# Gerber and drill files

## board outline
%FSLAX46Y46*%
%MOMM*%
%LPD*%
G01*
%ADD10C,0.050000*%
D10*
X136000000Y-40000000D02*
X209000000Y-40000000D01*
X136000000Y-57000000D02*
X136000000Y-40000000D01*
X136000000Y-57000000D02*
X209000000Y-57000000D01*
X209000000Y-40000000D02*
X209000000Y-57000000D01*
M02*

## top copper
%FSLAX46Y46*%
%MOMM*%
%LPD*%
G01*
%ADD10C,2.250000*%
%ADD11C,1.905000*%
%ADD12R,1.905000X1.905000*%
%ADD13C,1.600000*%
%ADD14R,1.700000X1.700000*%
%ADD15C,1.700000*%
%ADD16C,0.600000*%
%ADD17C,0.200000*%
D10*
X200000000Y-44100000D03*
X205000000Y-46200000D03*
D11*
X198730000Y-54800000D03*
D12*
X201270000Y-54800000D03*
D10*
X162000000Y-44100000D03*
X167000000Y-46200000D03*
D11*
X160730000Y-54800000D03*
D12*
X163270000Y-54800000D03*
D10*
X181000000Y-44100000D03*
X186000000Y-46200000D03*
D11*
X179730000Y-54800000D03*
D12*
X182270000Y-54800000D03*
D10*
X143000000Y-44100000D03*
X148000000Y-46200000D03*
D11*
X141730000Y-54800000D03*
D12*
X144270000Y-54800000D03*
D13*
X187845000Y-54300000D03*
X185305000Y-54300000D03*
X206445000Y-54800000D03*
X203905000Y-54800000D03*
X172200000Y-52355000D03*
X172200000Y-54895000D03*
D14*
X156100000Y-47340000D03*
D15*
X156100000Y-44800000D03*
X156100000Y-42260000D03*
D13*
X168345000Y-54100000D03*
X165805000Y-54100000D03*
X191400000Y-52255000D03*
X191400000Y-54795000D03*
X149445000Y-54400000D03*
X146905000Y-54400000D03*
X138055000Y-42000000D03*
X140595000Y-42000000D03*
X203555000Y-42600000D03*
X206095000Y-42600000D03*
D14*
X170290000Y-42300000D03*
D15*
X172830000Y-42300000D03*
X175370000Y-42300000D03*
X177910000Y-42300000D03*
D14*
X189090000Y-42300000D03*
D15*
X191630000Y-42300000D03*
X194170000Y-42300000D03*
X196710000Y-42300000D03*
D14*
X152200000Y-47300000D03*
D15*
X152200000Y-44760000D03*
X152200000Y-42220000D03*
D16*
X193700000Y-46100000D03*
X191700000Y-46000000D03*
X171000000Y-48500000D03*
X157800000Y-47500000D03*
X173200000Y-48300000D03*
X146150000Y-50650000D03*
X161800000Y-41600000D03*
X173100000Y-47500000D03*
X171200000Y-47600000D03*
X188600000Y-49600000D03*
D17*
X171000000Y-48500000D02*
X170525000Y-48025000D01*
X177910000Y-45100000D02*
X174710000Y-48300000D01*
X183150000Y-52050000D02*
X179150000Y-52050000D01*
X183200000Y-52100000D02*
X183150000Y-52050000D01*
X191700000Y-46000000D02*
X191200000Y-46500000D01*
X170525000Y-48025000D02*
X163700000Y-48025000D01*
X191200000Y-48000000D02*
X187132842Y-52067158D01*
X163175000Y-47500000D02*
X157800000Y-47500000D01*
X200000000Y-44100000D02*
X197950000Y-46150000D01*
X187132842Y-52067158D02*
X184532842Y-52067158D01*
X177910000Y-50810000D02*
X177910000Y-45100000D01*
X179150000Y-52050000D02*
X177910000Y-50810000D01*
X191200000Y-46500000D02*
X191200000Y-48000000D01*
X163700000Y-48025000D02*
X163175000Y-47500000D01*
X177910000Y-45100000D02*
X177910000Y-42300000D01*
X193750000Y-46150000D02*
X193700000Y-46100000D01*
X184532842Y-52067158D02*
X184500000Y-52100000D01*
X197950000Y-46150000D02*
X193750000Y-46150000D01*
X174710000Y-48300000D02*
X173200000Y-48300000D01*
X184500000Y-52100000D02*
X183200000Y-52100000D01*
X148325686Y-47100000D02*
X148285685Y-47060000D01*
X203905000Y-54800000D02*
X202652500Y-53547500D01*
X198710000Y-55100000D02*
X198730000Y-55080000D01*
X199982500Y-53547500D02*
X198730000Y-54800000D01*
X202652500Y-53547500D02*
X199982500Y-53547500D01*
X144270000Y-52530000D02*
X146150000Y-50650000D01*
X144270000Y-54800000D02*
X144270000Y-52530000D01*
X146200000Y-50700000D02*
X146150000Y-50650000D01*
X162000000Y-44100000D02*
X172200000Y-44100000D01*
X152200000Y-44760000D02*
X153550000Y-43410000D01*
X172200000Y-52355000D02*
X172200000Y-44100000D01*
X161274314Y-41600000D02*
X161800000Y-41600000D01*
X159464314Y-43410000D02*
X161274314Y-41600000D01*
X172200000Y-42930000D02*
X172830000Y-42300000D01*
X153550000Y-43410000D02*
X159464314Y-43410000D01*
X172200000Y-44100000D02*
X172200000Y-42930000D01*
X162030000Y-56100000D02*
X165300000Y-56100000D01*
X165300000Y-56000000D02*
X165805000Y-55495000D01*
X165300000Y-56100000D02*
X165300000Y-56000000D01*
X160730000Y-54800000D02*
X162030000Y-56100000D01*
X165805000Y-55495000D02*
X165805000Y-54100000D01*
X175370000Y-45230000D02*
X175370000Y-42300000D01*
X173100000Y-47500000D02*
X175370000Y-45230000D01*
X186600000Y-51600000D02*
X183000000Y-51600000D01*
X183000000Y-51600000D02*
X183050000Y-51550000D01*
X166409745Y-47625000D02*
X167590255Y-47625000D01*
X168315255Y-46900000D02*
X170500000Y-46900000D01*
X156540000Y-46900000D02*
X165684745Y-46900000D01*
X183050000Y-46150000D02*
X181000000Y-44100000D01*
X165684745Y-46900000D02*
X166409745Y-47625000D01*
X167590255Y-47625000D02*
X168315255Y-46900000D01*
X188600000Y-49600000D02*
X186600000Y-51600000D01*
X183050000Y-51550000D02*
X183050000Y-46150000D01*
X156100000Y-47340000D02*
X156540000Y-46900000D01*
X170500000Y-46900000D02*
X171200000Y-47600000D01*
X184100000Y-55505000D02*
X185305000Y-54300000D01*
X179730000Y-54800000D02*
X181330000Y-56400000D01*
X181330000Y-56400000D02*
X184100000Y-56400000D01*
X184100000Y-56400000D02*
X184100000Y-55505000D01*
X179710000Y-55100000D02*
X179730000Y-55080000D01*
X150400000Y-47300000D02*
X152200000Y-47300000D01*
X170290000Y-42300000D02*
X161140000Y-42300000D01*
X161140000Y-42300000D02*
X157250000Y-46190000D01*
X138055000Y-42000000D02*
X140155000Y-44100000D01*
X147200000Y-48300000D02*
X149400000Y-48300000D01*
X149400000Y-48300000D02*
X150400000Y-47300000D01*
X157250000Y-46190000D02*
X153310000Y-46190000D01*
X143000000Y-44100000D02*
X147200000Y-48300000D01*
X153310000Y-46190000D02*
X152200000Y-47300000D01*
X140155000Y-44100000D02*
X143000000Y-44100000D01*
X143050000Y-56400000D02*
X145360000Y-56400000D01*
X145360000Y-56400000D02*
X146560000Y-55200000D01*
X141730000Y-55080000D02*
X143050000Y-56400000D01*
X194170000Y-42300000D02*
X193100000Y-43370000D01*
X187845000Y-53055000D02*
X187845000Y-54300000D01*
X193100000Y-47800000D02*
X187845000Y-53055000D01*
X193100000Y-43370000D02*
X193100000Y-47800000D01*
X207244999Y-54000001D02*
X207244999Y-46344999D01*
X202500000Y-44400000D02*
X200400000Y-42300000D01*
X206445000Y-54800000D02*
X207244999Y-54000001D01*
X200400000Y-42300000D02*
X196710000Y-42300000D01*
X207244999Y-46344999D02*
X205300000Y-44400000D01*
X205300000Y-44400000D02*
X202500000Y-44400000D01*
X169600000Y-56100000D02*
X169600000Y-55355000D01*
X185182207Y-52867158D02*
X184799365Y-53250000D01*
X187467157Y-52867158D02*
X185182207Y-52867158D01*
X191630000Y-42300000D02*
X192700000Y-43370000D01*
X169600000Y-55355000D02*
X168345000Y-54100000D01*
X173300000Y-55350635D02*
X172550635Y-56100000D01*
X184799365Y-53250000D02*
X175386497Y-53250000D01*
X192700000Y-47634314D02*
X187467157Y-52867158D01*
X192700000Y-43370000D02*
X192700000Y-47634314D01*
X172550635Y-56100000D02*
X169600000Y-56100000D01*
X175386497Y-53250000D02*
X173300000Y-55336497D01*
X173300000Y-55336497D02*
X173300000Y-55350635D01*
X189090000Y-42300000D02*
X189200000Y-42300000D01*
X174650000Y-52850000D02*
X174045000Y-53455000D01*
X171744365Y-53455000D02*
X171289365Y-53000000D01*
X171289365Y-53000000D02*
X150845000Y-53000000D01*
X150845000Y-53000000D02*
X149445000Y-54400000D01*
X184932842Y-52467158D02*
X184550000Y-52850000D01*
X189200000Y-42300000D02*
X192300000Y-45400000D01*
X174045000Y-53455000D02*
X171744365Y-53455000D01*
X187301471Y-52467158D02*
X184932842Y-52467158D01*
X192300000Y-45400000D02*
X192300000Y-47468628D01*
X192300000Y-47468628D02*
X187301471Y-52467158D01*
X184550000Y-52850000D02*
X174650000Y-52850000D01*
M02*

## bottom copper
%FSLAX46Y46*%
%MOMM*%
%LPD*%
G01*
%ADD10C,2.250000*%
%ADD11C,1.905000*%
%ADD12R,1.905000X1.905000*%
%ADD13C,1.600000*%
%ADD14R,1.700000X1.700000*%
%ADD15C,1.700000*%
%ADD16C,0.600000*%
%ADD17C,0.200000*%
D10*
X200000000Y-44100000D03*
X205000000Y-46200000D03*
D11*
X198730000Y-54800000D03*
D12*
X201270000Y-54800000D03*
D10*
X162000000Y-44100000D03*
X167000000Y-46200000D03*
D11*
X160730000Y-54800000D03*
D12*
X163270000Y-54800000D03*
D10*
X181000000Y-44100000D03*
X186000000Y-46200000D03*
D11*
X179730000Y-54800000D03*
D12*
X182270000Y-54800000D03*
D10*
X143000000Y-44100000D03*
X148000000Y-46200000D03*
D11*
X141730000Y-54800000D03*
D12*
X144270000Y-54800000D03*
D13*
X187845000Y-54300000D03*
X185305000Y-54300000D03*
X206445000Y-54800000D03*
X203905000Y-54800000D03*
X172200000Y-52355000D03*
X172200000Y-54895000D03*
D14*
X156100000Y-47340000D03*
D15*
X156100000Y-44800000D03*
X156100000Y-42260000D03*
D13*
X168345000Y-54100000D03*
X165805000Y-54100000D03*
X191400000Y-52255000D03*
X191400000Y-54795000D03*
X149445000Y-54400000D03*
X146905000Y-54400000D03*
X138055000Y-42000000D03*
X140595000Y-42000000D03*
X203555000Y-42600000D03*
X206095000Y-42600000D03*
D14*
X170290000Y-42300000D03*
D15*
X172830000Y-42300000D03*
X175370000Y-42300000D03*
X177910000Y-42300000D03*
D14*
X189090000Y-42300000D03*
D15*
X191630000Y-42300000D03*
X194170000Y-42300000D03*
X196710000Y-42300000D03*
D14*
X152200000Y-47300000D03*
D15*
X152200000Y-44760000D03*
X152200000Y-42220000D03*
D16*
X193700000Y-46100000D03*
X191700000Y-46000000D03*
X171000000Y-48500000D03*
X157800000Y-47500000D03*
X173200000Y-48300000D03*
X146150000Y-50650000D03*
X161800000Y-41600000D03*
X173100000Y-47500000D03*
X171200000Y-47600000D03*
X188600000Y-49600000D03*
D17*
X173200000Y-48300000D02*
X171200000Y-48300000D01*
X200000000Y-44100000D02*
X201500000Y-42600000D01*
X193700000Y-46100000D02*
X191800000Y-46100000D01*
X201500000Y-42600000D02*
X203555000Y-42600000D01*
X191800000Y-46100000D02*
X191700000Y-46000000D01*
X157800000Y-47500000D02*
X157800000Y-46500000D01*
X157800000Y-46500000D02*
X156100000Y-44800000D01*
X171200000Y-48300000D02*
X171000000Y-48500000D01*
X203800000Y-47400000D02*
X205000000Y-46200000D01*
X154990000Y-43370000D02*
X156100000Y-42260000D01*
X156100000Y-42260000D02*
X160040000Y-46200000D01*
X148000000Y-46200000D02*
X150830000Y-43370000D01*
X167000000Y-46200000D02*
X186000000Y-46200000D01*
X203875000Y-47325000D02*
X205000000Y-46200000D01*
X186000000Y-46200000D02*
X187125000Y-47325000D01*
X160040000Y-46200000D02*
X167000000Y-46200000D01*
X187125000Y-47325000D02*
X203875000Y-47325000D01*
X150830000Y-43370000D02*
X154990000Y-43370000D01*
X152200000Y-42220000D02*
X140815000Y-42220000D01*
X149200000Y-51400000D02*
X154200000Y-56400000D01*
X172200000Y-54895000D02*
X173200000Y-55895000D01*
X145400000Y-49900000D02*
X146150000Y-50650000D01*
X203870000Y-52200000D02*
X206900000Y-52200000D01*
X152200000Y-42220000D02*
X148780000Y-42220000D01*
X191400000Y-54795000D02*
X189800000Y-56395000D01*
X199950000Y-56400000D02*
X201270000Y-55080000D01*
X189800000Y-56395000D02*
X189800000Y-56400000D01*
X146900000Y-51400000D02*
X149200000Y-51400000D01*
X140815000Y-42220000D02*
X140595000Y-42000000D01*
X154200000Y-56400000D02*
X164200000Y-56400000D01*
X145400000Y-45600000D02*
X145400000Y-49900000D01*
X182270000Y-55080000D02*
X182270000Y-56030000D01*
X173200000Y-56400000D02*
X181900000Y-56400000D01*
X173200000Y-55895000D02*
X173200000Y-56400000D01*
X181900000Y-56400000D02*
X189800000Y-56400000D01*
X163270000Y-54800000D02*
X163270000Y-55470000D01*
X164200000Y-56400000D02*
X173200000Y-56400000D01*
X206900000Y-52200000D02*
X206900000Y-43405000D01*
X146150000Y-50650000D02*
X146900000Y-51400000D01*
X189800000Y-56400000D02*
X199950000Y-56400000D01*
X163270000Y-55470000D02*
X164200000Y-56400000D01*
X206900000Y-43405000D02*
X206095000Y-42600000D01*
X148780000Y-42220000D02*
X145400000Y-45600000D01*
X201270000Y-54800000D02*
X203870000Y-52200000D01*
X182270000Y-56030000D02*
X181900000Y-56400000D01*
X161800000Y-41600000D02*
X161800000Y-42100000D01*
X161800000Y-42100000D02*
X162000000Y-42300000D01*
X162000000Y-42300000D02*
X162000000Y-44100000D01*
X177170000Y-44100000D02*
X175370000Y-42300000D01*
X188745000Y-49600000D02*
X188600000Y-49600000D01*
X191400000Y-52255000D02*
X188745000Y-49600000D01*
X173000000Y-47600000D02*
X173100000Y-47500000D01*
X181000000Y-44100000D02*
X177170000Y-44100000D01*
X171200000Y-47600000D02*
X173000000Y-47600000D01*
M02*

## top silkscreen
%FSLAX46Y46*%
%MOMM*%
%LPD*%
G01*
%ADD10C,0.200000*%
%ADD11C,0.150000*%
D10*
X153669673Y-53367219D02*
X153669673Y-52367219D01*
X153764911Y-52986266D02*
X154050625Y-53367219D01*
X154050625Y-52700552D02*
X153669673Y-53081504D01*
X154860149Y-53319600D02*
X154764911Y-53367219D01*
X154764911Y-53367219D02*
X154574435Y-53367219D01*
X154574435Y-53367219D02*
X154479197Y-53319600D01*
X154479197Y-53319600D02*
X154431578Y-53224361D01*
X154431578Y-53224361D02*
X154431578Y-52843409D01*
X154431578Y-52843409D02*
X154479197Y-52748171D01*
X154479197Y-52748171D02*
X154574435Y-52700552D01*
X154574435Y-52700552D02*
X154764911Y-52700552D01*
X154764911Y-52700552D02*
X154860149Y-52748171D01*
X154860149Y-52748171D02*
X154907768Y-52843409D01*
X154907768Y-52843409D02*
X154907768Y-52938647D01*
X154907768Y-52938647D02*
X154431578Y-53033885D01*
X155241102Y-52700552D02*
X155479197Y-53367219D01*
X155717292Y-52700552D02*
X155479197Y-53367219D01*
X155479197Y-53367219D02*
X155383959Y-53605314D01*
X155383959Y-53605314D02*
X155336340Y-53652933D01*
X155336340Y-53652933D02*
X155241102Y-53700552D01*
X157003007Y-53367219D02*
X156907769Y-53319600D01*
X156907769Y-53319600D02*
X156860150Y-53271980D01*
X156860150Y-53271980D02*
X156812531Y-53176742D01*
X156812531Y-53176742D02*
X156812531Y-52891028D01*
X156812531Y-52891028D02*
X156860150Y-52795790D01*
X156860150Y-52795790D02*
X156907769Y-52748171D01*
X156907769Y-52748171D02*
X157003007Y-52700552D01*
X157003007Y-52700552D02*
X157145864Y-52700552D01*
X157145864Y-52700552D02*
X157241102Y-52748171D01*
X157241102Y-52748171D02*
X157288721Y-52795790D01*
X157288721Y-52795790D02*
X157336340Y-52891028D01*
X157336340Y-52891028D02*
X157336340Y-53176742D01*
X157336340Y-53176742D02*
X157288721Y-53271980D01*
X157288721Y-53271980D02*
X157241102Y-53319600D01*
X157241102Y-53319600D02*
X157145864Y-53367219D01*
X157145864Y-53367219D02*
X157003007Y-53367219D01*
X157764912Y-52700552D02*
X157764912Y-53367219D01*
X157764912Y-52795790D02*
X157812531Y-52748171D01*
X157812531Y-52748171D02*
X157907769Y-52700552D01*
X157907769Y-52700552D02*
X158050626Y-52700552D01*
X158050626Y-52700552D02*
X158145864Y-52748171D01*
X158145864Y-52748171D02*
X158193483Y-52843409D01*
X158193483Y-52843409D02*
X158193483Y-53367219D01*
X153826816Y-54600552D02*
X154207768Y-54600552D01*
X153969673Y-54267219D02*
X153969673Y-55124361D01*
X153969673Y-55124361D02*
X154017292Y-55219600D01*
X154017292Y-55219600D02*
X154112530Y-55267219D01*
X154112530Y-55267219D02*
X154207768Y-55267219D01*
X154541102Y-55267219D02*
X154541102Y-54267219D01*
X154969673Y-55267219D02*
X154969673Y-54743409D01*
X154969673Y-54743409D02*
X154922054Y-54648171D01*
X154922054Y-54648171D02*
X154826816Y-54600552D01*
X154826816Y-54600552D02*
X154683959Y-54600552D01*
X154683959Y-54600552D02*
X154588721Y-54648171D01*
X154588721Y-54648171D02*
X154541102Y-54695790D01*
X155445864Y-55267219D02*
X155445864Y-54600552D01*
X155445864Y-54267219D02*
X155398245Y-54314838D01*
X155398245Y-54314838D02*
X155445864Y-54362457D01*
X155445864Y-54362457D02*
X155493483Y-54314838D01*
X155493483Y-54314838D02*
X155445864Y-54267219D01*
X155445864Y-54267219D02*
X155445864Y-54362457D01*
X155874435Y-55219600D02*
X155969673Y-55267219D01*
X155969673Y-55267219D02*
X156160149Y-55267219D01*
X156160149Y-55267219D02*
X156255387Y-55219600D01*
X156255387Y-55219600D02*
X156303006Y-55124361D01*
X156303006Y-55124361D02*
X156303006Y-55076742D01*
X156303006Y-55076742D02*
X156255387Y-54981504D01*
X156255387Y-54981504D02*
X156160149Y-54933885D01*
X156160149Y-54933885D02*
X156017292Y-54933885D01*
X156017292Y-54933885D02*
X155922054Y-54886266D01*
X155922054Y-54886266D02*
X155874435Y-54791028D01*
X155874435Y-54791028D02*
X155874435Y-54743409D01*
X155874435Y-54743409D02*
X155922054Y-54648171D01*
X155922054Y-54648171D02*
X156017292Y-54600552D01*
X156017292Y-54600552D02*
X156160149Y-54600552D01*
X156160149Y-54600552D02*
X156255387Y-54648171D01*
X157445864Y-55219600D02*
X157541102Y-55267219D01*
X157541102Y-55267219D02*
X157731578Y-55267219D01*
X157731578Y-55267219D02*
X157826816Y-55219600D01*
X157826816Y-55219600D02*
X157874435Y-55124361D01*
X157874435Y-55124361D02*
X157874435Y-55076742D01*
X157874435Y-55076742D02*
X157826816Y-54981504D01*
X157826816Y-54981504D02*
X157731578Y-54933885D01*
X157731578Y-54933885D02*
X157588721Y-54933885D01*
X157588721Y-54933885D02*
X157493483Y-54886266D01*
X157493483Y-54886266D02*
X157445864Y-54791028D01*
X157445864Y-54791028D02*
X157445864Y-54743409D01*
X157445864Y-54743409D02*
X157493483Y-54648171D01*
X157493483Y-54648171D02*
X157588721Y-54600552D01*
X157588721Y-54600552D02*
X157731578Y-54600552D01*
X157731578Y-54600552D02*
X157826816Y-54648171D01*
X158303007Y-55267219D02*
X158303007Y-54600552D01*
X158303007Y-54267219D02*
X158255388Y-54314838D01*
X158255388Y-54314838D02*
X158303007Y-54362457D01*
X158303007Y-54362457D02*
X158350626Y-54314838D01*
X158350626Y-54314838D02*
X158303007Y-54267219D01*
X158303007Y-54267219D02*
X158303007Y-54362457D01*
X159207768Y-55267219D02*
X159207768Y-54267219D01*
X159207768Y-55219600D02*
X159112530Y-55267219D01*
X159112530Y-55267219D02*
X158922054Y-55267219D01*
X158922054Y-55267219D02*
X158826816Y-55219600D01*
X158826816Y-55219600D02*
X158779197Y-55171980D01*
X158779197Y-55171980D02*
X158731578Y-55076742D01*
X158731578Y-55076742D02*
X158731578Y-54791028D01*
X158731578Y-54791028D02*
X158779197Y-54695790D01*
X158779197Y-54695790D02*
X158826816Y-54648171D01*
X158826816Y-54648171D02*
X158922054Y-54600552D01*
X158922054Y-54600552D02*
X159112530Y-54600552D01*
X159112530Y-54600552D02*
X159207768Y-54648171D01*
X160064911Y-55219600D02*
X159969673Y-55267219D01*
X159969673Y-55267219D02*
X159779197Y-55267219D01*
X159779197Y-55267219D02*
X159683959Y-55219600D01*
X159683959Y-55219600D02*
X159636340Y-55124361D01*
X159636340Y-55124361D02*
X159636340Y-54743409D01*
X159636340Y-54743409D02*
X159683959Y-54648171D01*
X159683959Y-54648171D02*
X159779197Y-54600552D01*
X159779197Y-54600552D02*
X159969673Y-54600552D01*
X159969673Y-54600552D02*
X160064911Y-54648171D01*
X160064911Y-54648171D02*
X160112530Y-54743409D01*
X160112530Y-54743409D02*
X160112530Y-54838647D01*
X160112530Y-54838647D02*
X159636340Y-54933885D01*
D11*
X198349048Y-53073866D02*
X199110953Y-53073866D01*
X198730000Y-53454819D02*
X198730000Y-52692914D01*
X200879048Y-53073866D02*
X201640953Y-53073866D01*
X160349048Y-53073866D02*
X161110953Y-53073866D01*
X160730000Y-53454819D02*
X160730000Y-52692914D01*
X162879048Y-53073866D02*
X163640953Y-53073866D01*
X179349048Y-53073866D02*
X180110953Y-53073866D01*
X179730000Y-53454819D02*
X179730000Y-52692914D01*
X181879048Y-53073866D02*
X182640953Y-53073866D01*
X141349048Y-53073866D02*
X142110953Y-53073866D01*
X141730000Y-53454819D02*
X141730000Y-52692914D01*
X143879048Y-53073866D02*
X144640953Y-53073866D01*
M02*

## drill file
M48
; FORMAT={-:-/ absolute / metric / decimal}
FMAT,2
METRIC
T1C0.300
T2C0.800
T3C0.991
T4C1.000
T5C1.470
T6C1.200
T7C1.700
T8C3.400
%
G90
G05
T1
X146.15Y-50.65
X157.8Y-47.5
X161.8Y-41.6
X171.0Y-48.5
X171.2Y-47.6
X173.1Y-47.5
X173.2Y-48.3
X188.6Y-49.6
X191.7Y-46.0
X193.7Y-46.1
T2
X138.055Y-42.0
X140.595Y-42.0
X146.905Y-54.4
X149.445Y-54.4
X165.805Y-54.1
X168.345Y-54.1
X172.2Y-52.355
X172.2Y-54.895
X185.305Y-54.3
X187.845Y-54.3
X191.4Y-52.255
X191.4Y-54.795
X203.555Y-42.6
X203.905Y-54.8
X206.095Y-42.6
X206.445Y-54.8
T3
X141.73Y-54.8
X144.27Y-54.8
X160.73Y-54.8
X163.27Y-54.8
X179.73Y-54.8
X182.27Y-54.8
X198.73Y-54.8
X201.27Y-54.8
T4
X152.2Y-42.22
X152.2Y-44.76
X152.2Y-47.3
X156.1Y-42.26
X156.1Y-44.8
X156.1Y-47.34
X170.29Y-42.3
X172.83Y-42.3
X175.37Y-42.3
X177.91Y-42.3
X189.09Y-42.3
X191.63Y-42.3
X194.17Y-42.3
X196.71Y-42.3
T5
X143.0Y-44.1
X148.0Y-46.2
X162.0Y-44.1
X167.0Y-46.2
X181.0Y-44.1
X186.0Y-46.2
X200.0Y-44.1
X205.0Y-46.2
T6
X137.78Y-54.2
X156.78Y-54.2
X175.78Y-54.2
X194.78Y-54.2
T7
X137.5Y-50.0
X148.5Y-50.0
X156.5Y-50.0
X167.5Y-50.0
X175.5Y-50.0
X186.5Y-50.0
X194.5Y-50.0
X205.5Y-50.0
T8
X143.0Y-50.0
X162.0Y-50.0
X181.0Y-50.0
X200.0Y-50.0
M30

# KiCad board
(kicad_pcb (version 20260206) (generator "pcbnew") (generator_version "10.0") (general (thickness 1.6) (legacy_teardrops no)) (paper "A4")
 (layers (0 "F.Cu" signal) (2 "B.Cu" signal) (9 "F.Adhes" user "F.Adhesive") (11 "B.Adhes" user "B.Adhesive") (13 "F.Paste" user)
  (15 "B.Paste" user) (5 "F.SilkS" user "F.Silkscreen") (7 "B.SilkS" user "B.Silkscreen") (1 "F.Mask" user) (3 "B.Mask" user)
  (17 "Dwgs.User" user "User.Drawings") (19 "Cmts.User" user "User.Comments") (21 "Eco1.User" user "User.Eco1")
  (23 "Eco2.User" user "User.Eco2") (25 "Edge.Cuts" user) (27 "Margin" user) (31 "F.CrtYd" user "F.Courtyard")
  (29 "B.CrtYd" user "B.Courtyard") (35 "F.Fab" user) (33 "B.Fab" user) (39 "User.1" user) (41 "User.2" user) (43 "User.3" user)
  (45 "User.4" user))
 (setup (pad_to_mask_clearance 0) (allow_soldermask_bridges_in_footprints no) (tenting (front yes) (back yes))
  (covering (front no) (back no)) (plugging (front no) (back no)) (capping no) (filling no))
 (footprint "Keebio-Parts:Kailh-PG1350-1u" (layer "F.Cu") (at 200 50 180)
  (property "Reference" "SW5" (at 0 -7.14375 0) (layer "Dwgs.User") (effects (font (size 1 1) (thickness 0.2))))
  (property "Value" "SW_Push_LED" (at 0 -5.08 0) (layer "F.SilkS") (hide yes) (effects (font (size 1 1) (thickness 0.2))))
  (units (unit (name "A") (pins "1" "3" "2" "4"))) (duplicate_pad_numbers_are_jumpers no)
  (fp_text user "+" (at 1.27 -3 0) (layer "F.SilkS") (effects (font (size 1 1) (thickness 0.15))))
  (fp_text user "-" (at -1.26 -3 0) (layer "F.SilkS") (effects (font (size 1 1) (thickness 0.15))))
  (pad "" np_thru_hole circle (at -5.5 0) (size 1.7 1.7) (drill 1.7) (layers "*.Cu" "*.Mask"))
  (pad "" np_thru_hole circle (at 0 0) (size 3.4 3.4) (drill 3.4) (layers "*.Cu" "*.Mask"))
  (pad "" np_thru_hole circle (at 5.22 -4.2) (size 1.2 1.2) (drill 1.2) (layers "*.Cu" "*.Mask"))
  (pad "" np_thru_hole circle (at 5.5 0) (size 1.7 1.7) (drill 1.7) (layers "*.Cu" "*.Mask"))
  (pad "1" thru_hole circle (at 0 5.9) (size 2.25 2.25) (drill 1.47) (layers "*.Cu" "*.Mask") (remove_unused_layers no) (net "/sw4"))
  (pad "2" thru_hole circle (at -5 3.8 221.9) (size 2.25 2.25) (drill 1.47) (layers "*.Cu" "*.Mask") (remove_unused_layers no) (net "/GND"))
  (pad "3" thru_hole circle (at 1.27 -4.8) (size 1.905 1.905) (drill 0.9906) (layers "*.Cu" "*.Mask") (remove_unused_layers no)
   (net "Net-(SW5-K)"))
  (pad "4" thru_hole rect (at -1.27 -4.8) (size 1.905 1.905) (drill 0.9906) (layers "*.Cu" "*.Mask") (remove_unused_layers no) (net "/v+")))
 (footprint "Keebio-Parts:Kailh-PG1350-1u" (layer "F.Cu") (at 162 50 180)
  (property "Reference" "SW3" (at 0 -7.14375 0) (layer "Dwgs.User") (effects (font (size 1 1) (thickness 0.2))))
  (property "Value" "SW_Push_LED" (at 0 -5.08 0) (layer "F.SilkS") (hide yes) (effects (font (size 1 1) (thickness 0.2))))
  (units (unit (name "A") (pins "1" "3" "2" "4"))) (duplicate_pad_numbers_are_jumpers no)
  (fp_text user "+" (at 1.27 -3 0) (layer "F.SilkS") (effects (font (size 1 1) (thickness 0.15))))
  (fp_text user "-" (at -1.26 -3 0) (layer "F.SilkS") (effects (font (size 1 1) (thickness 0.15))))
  (pad "" np_thru_hole circle (at -5.5 0) (size 1.7 1.7) (drill 1.7) (layers "*.Cu" "*.Mask"))
  (pad "" np_thru_hole circle (at 0 0) (size 3.4 3.4) (drill 3.4) (layers "*.Cu" "*.Mask"))
  (pad "" np_thru_hole circle (at 5.22 -4.2) (size 1.2 1.2) (drill 1.2) (layers "*.Cu" "*.Mask"))
  (pad "" np_thru_hole circle (at 5.5 0) (size 1.7 1.7) (drill 1.7) (layers "*.Cu" "*.Mask"))
  (pad "1" thru_hole circle (at 0 5.9) (size 2.25 2.25) (drill 1.47) (layers "*.Cu" "*.Mask") (remove_unused_layers no) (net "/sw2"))
  (pad "2" thru_hole circle (at -5 3.8 221.9) (size 2.25 2.25) (drill 1.47) (layers "*.Cu" "*.Mask") (remove_unused_layers no) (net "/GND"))
  (pad "3" thru_hole circle (at 1.27 -4.8) (size 1.905 1.905) (drill 0.9906) (layers "*.Cu" "*.Mask") (remove_unused_layers no)
   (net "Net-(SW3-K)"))
  (pad "4" thru_hole rect (at -1.27 -4.8) (size 1.905 1.905) (drill 0.9906) (layers "*.Cu" "*.Mask") (remove_unused_layers no) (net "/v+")))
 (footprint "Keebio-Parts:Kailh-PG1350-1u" (layer "F.Cu") (at 181 50 180)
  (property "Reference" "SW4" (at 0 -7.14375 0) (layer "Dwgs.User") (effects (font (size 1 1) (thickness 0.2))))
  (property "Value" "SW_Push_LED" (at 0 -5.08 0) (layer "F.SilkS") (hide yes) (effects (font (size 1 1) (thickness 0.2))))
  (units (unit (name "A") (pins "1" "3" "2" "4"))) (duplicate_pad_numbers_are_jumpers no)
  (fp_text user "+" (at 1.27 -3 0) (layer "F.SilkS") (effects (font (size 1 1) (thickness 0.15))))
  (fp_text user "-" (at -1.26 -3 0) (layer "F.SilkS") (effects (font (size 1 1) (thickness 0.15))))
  (pad "" np_thru_hole circle (at -5.5 0) (size 1.7 1.7) (drill 1.7) (layers "*.Cu" "*.Mask"))
  (pad "" np_thru_hole circle (at 0 0) (size 3.4 3.4) (drill 3.4) (layers "*.Cu" "*.Mask"))
  (pad "" np_thru_hole circle (at 5.22 -4.2) (size 1.2 1.2) (drill 1.2) (layers "*.Cu" "*.Mask"))
  (pad "" np_thru_hole circle (at 5.5 0) (size 1.7 1.7) (drill 1.7) (layers "*.Cu" "*.Mask"))
  (pad "1" thru_hole circle (at 0 5.9) (size 2.25 2.25) (drill 1.47) (layers "*.Cu" "*.Mask") (remove_unused_layers no) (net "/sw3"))
  (pad "2" thru_hole circle (at -5 3.8 221.9) (size 2.25 2.25) (drill 1.47) (layers "*.Cu" "*.Mask") (remove_unused_layers no) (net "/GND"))
  (pad "3" thru_hole circle (at 1.27 -4.8) (size 1.905 1.905) (drill 0.9906) (layers "*.Cu" "*.Mask") (remove_unused_layers no)
   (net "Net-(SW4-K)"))
  (pad "4" thru_hole rect (at -1.27 -4.8) (size 1.905 1.905) (drill 0.9906) (layers "*.Cu" "*.Mask") (remove_unused_layers no) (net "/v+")))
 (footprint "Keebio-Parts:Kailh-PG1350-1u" (layer "F.Cu") (at 143 50 180)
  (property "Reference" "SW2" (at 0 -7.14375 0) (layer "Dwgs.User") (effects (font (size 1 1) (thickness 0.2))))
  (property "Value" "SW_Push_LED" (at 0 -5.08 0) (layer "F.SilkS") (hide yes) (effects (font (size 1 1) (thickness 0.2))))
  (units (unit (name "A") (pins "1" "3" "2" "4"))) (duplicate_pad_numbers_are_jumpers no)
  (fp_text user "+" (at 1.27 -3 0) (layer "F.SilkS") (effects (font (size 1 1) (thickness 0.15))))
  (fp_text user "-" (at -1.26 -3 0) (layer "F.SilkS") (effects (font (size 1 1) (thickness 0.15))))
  (pad "" np_thru_hole circle (at -5.5 0) (size 1.7 1.7) (drill 1.7) (layers "*.Cu" "*.Mask"))
  (pad "" np_thru_hole circle (at 0 0) (size 3.4 3.4) (drill 3.4) (layers "*.Cu" "*.Mask"))
  (pad "" np_thru_hole circle (at 5.22 -4.2) (size 1.2 1.2) (drill 1.2) (layers "*.Cu" "*.Mask"))
  (pad "" np_thru_hole circle (at 5.5 0) (size 1.7 1.7) (drill 1.7) (layers "*.Cu" "*.Mask"))
  (pad "1" thru_hole circle (at 0 5.9) (size 2.25 2.25) (drill 1.47) (layers "*.Cu" "*.Mask") (remove_unused_layers no) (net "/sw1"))
  (pad "2" thru_hole circle (at -5 3.8 221.9) (size 2.25 2.25) (drill 1.47) (layers "*.Cu" "*.Mask") (remove_unused_layers no) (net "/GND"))
  (pad "3" thru_hole circle (at 1.27 -4.8) (size 1.905 1.905) (drill 0.9906) (layers "*.Cu" "*.Mask") (remove_unused_layers no)
   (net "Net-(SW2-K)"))
  (pad "4" thru_hole rect (at -1.27 -4.8) (size 1.905 1.905) (drill 0.9906) (layers "*.Cu" "*.Mask") (remove_unused_layers no) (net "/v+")))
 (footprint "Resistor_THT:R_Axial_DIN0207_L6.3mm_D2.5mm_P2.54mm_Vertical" (layer "B.Cu") (at 187.845 54.3 180)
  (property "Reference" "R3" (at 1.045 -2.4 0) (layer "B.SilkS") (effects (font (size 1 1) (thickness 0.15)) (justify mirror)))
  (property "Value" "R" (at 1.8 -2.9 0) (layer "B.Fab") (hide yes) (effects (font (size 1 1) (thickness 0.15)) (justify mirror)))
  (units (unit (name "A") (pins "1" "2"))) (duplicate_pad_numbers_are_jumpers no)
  (pad "1" thru_hole circle (at 0 0 180) (size 1.6 1.6) (drill 0.8) (layers "*.Cu" "*.Mask") (remove_unused_layers no) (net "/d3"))
  (pad "2" thru_hole circle (at 2.54 0 180) (size 1.6 1.6) (drill 0.8) (layers "*.Cu" "*.Mask") (remove_unused_layers no)
   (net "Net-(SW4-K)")))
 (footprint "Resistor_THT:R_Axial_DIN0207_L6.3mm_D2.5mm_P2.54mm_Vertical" (layer "B.Cu") (at 206.445 54.8 180)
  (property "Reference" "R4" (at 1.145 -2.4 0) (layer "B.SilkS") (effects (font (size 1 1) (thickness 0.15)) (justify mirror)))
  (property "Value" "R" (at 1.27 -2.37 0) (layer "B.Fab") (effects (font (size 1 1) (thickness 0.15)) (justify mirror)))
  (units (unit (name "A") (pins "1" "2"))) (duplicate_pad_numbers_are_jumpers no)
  (pad "1" thru_hole circle (at 0 0 180) (size 1.6 1.6) (drill 0.8) (layers "*.Cu" "*.Mask") (remove_unused_layers no) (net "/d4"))
  (pad "2" thru_hole circle (at 2.54 0 180) (size 1.6 1.6) (drill 0.8) (layers "*.Cu" "*.Mask") (remove_unused_layers no)
   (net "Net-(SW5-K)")))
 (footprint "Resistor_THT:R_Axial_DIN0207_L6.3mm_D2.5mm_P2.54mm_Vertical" (layer "B.Cu") (at 172.2 52.355 -90)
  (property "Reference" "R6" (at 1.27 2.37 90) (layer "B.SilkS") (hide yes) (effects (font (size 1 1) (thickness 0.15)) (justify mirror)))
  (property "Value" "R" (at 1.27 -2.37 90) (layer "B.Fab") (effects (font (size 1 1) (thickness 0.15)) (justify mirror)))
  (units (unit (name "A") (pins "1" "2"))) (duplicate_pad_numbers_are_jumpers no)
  (pad "1" thru_hole circle (at 0 0 270) (size 1.6 1.6) (drill 0.8) (layers "*.Cu" "*.Mask") (remove_unused_layers no) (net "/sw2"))
  (pad "2" thru_hole circle (at 2.54 0 270) (size 1.6 1.6) (drill 0.8) (layers "*.Cu" "*.Mask") (remove_unused_layers no) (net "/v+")))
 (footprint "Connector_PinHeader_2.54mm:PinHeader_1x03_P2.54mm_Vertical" (layer "B.Cu") (at 156.1 47.34)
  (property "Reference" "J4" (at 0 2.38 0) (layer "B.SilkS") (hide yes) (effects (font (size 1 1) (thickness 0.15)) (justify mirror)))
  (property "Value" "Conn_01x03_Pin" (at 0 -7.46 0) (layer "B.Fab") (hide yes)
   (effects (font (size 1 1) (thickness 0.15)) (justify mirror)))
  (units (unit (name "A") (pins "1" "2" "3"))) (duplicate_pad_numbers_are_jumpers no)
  (pad "1" thru_hole rect (at 0 0) (size 1.7 1.7) (drill 1) (layers "*.Cu" "*.Mask") (remove_unused_layers no) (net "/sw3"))
  (pad "2" thru_hole circle (at 0 -2.54) (size 1.7 1.7) (drill 1) (layers "*.Cu" "*.Mask") (remove_unused_layers no) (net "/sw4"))
  (pad "3" thru_hole circle (at 0 -5.08) (size 1.7 1.7) (drill 1) (layers "*.Cu" "*.Mask") (remove_unused_layers no) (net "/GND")))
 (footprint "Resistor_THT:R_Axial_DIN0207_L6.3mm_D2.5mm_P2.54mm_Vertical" (layer "B.Cu") (at 168.345 54.1 180)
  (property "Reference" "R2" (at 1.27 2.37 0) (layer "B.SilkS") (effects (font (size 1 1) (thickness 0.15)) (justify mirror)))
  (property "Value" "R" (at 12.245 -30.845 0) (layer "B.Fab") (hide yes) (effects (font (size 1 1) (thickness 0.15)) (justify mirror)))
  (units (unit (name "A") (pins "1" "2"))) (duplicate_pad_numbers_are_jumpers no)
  (pad "1" thru_hole circle (at 0 0 180) (size 1.6 1.6) (drill 0.8) (layers "*.Cu" "*.Mask") (remove_unused_layers no) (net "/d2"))
  (pad "2" thru_hole circle (at 2.54 0 180) (size 1.6 1.6) (drill 0.8) (layers "*.Cu" "*.Mask") (remove_unused_layers no)
   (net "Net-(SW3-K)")))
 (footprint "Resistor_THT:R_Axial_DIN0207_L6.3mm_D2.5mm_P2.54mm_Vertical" (layer "B.Cu") (at 191.4 52.255 -90)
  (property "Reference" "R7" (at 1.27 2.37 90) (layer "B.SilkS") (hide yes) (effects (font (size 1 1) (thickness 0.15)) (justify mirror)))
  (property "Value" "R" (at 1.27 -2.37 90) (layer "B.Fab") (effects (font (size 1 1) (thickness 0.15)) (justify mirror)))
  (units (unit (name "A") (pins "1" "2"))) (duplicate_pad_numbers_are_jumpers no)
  (pad "1" thru_hole circle (at 0 0 270) (size 1.6 1.6) (drill 0.8) (layers "*.Cu" "*.Mask") (remove_unused_layers no) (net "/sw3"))
  (pad "2" thru_hole circle (at 2.54 0 270) (size 1.6 1.6) (drill 0.8) (layers "*.Cu" "*.Mask") (remove_unused_layers no) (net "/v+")))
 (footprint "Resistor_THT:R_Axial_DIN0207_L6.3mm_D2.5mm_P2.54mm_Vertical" (layer "B.Cu") (at 149.445 54.4 180)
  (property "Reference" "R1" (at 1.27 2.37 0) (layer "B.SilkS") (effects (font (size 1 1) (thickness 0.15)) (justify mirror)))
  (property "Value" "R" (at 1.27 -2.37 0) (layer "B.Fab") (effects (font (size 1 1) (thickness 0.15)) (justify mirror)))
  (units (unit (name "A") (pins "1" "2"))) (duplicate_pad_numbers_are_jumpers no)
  (pad "1" thru_hole circle (at 0 0 180) (size 1.6 1.6) (drill 0.8) (layers "*.Cu" "*.Mask") (remove_unused_layers no) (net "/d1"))
  (pad "2" thru_hole circle (at 2.54 0 180) (size 1.6 1.6) (drill 0.8) (layers "*.Cu" "*.Mask") (remove_unused_layers no)
   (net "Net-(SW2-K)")))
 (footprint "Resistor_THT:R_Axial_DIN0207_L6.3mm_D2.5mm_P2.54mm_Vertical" (layer "B.Cu") (at 138.055 42)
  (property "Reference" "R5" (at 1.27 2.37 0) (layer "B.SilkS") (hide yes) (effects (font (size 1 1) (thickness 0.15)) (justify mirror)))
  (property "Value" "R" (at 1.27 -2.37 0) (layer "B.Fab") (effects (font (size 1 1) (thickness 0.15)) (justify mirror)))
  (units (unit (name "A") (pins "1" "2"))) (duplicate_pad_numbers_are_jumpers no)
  (pad "1" thru_hole circle (at 0 0) (size 1.6 1.6) (drill 0.8) (layers "*.Cu" "*.Mask") (remove_unused_layers no) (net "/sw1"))
  (pad "2" thru_hole circle (at 2.54 0) (size 1.6 1.6) (drill 0.8) (layers "*.Cu" "*.Mask") (remove_unused_layers no) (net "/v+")))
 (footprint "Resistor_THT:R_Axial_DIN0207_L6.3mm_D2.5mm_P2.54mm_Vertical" (layer "B.Cu") (at 203.555 42.6)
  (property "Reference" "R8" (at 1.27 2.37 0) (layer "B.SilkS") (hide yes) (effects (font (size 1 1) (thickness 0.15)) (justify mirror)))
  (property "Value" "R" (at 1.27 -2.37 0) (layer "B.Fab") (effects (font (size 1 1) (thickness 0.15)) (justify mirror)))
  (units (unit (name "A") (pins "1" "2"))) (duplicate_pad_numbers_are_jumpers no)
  (pad "1" thru_hole circle (at 0 0) (size 1.6 1.6) (drill 0.8) (layers "*.Cu" "*.Mask") (remove_unused_layers no) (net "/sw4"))
  (pad "2" thru_hole circle (at 2.54 0) (size 1.6 1.6) (drill 0.8) (layers "*.Cu" "*.Mask") (remove_unused_layers no) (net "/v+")))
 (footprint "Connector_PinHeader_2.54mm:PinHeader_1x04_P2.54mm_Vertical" (layer "B.Cu") (at 170.29 42.3 -90)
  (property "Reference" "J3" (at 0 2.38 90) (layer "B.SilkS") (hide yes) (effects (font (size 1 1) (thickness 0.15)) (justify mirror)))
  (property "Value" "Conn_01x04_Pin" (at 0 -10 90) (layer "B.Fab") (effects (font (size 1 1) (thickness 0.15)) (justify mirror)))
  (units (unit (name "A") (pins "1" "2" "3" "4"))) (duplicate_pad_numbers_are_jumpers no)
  (pad "1" thru_hole rect (at 0 0 270) (size 1.7 1.7) (drill 1) (layers "*.Cu" "*.Mask") (remove_unused_layers no) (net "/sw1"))
  (pad "2" thru_hole circle (at 0 -2.54 270) (size 1.7 1.7) (drill 1) (layers "*.Cu" "*.Mask") (remove_unused_layers no) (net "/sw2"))
  (pad "3" thru_hole circle (at 0 -5.08 270) (size 1.7 1.7) (drill 1) (layers "*.Cu" "*.Mask") (remove_unused_layers no) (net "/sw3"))
  (pad "4" thru_hole circle (at 0 -7.62 270) (size 1.7 1.7) (drill 1) (layers "*.Cu" "*.Mask") (remove_unused_layers no) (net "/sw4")))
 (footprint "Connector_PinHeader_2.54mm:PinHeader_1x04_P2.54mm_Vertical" (layer "B.Cu") (at 189.09 42.3 -90)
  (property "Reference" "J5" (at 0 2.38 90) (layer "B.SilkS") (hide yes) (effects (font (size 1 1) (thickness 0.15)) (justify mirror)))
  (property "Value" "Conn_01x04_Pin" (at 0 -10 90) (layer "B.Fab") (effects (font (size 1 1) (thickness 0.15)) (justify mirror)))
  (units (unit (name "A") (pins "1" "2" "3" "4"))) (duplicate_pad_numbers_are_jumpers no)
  (pad "1" thru_hole rect (at 0 0 270) (size 1.7 1.7) (drill 1) (layers "*.Cu" "*.Mask") (remove_unused_layers no) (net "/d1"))
  (pad "2" thru_hole circle (at 0 -2.54 270) (size 1.7 1.7) (drill 1) (layers "*.Cu" "*.Mask") (remove_unused_layers no) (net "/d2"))
  (pad "3" thru_hole circle (at 0 -5.08 270) (size 1.7 1.7) (drill 1) (layers "*.Cu" "*.Mask") (remove_unused_layers no) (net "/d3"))
  (pad "4" thru_hole circle (at 0 -7.62 270) (size 1.7 1.7) (drill 1) (layers "*.Cu" "*.Mask") (remove_unused_layers no) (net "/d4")))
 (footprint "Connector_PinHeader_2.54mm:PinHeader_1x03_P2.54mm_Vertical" (layer "B.Cu") (at 152.2 47.3)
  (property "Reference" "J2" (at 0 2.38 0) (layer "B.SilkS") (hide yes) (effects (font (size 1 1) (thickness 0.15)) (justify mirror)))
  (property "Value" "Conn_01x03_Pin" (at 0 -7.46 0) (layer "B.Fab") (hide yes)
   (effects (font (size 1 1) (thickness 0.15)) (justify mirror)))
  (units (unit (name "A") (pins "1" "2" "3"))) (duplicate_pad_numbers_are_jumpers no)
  (pad "1" thru_hole rect (at 0 0) (size 1.7 1.7) (drill 1) (layers "*.Cu" "*.Mask") (remove_unused_layers no) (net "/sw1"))
  (pad "2" thru_hole circle (at 0 -2.54) (size 1.7 1.7) (drill 1) (layers "*.Cu" "*.Mask") (remove_unused_layers no) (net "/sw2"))
  (pad "3" thru_hole circle (at 0 -5.08) (size 1.7 1.7) (drill 1) (layers "*.Cu" "*.Mask") (remove_unused_layers no) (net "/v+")))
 (gr_line (start 136 40) (end 209 40) (stroke (width 0.05) (type solid)) (layer "Edge.Cuts"))
 (gr_line (start 136 57) (end 136 40) (stroke (width 0.05) (type default)) (layer "Edge.Cuts"))
 (gr_line (start 136 57) (end 209 57) (stroke (width 0.05) (type solid)) (layer "Edge.Cuts"))
 (gr_line (start 209 40) (end 209 57) (stroke (width 0.05) (type solid)) (layer "Edge.Cuts"))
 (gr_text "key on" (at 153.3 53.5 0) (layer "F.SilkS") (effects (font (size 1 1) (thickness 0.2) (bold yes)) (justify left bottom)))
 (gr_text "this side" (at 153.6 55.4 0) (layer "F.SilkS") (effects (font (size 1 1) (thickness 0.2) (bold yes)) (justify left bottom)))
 (segment (start 171 48.5) (end 170.525 48.025) (width 0.2) (layer "F.Cu") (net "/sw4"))
 (segment (start 177.91 45.1) (end 174.71 48.3) (width 0.2) (layer "F.Cu") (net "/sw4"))
 (segment (start 183.15 52.05) (end 179.15 52.05) (width 0.2) (layer "F.Cu") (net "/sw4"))
 (segment (start 183.2 52.1) (end 183.15 52.05) (width 0.2) (layer "F.Cu") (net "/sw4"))
 (segment (start 191.7 46) (end 191.2 46.5) (width 0.2) (layer "F.Cu") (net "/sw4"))
 (segment (start 170.525 48.025) (end 163.7 48.025) (width 0.2) (layer "F.Cu") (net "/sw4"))
 (segment (start 191.2 48) (end 187.132842 52.067158) (width 0.2) (layer "F.Cu") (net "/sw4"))
 (segment (start 163.175 47.5) (end 157.8 47.5) (width 0.2) (layer "F.Cu") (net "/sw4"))
 (segment (start 200 44.1) (end 197.95 46.15) (width 0.2) (layer "F.Cu") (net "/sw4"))
 (segment (start 187.132842 52.067158) (end 184.532842 52.067158) (width 0.2) (layer "F.Cu") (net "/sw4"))
 (segment (start 177.91 50.81) (end 177.91 45.1) (width 0.2) (layer "F.Cu") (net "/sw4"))
 (segment (start 179.15 52.05) (end 177.91 50.81) (width 0.2) (layer "F.Cu") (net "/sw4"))
 (segment (start 191.2 46.5) (end 191.2 48) (width 0.2) (layer "F.Cu") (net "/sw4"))
 (segment (start 163.7 48.025) (end 163.175 47.5) (width 0.2) (layer "F.Cu") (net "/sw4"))
 (segment (start 177.91 45.1) (end 177.91 42.3) (width 0.2) (layer "F.Cu") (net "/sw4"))
 (segment (start 193.75 46.15) (end 193.7 46.1) (width 0.2) (layer "F.Cu") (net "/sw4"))
 (segment (start 184.532842 52.067158) (end 184.5 52.1) (width 0.2) (layer "F.Cu") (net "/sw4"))
 (segment (start 197.95 46.15) (end 193.75 46.15) (width 0.2) (layer "F.Cu") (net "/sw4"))
 (segment (start 174.71 48.3) (end 173.2 48.3) (width 0.2) (layer "F.Cu") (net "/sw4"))
 (segment (start 184.5 52.1) (end 183.2 52.1) (width 0.2) (layer "F.Cu") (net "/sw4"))
 (via (at 193.7 46.1) (size 0.6) (drill 0.3) (layers "F.Cu" "B.Cu") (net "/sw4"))
 (via (at 191.7 46) (size 0.6) (drill 0.3) (layers "F.Cu" "B.Cu") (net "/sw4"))
 (via (at 171 48.5) (size 0.6) (drill 0.3) (layers "F.Cu" "B.Cu") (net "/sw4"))
 (via (at 157.8 47.5) (size 0.6) (drill 0.3) (layers "F.Cu" "B.Cu") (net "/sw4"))
 (via (at 173.2 48.3) (size 0.6) (drill 0.3) (layers "F.Cu" "B.Cu") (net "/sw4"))
 (segment (start 173.2 48.3) (end 171.2 48.3) (width 0.2) (layer "B.Cu") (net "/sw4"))
 (segment (start 200 44.1) (end 201.5 42.6) (width 0.2) (layer "B.Cu") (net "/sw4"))
 (segment (start 193.7 46.1) (end 191.8 46.1) (width 0.2) (layer "B.Cu") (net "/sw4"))
 (segment (start 201.5 42.6) (end 203.555 42.6) (width 0.2) (layer "B.Cu") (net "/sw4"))
 (segment (start 191.8 46.1) (end 191.7 46) (width 0.2) (layer "B.Cu") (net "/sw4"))
 (segment (start 157.8 47.5) (end 157.8 46.5) (width 0.2) (layer "B.Cu") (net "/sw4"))
 (segment (start 157.8 46.5) (end 156.1 44.8) (width 0.2) (layer "B.Cu") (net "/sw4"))
 (segment (start 171.2 48.3) (end 171 48.5) (width 0.2) (layer "B.Cu") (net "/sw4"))
 (segment (start 148.325686 47.1) (end 148.285685 47.06) (width 0.2) (layer "F.Cu") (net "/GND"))
 (segment (start 203.8 47.4) (end 205 46.2) (width 0.2) (layer "B.Cu") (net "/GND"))
 (segment (start 154.99 43.37) (end 156.1 42.26) (width 0.2) (layer "B.Cu") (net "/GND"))
 (segment (start 156.1 42.26) (end 160.04 46.2) (width 0.2) (layer "B.Cu") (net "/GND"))
 (segment (start 148 46.2) (end 150.83 43.37) (width 0.2) (layer "B.Cu") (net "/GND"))
 (segment (start 167 46.2) (end 186 46.2) (width 0.2) (layer "B.Cu") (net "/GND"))
 (segment (start 203.875 47.325) (end 205 46.2) (width 0.2) (layer "B.Cu") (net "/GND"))
 (segment (start 186 46.2) (end 187.125 47.325) (width 0.2) (layer "B.Cu") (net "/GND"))
 (segment (start 160.04 46.2) (end 167 46.2) (width 0.2) (layer "B.Cu") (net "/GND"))
 (segment (start 187.125 47.325) (end 203.875 47.325) (width 0.2) (layer "B.Cu") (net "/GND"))
 (segment (start 150.83 43.37) (end 154.99 43.37) (width 0.2) (layer "B.Cu") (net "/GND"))
 (segment (start 203.905 54.8) (end 202.6525 53.5475) (width 0.2) (layer "F.Cu") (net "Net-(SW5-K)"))
 (segment (start 198.71 55.1) (end 198.73 55.08) (width 0.2) (layer "F.Cu") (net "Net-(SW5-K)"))
 (segment (start 199.9825 53.5475) (end 198.73 54.8) (width 0.2) (layer "F.Cu") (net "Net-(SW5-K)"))
 (segment (start 202.6525 53.5475) (end 199.9825 53.5475) (width 0.2) (layer "F.Cu") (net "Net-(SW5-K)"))
 (segment (start 144.27 52.53) (end 146.15 50.65) (width 0.2) (layer "F.Cu") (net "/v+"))
 (segment (start 144.27 54.8) (end 144.27 52.53) (width 0.2) (layer "F.Cu") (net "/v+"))
 (segment (start 146.2 50.7) (end 146.15 50.65) (width 0.2) (layer "F.Cu") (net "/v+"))
 (via (at 146.15 50.65) (size 0.6) (drill 0.3) (layers "F.Cu" "B.Cu") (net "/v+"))
 (segment (start 152.2 42.22) (end 140.815 42.22) (width 0.2) (layer "B.Cu") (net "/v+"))
 (segment (start 149.2 51.4) (end 154.2 56.4) (width 0.2) (layer "B.Cu") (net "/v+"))
 (segment (start 172.2 54.895) (end 173.2 55.895) (width 0.2) (layer "B.Cu") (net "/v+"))
 (segment (start 145.4 49.9) (end 146.15 50.65) (width 0.2) (layer "B.Cu") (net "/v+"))
 (segment (start 203.87 52.2) (end 206.9 52.2) (width 0.2) (layer "B.Cu") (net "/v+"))
 (segment (start 152.2 42.22) (end 148.78 42.22) (width 0.2) (layer "B.Cu") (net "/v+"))
 (segment (start 191.4 54.795) (end 189.8 56.395) (width 0.2) (layer "B.Cu") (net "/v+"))
 (segment (start 199.95 56.4) (end 201.27 55.08) (width 0.2) (layer "B.Cu") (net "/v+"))
 (segment (start 189.8 56.395) (end 189.8 56.4) (width 0.2) (layer "B.Cu") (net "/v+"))
 (segment (start 146.9 51.4) (end 149.2 51.4) (width 0.2) (layer "B.Cu") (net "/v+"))
 (segment (start 140.815 42.22) (end 140.595 42) (width 0.2) (layer "B.Cu") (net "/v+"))
 (segment (start 154.2 56.4) (end 164.2 56.4) (width 0.2) (layer "B.Cu") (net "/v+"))
 (segment (start 145.4 45.6) (end 145.4 49.9) (width 0.2) (layer "B.Cu") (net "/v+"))
 (segment (start 182.27 55.08) (end 182.27 56.03) (width 0.2) (layer "B.Cu") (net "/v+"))
 (segment (start 173.2 56.4) (end 181.9 56.4) (width 0.2) (layer "B.Cu") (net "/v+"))
 (segment (start 173.2 55.895) (end 173.2 56.4) (width 0.2) (layer "B.Cu") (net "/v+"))
 (segment (start 181.9 56.4) (end 189.8 56.4) (width 0.2) (layer "B.Cu") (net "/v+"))
 (segment (start 163.27 54.8) (end 163.27 55.47) (width 0.2) (layer "B.Cu") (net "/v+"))
 (segment (start 164.2 56.4) (end 173.2 56.4) (width 0.2) (layer "B.Cu") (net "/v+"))
 (segment (start 206.9 52.2) (end 206.9 43.405) (width 0.2) (layer "B.Cu") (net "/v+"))
 (segment (start 146.15 50.65) (end 146.9 51.4) (width 0.2) (layer "B.Cu") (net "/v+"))
 (segment (start 189.8 56.4) (end 199.95 56.4) (width 0.2) (layer "B.Cu") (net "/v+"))
 (segment (start 163.27 55.47) (end 164.2 56.4) (width 0.2) (layer "B.Cu") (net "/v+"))
 (segment (start 206.9 43.405) (end 206.095 42.6) (width 0.2) (layer "B.Cu") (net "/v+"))
 (segment (start 148.78 42.22) (end 145.4 45.6) (width 0.2) (layer "B.Cu") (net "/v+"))
 (segment (start 201.27 54.8) (end 203.87 52.2) (width 0.2) (layer "B.Cu") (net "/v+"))
 (segment (start 182.27 56.03) (end 181.9 56.4) (width 0.2) (layer "B.Cu") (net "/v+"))
 (segment (start 162 44.1) (end 172.2 44.1) (width 0.2) (layer "F.Cu") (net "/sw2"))
 (segment (start 152.2 44.76) (end 153.55 43.41) (width 0.2) (layer "F.Cu") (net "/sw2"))
 (segment (start 172.2 52.355) (end 172.2 44.1) (width 0.2) (layer "F.Cu") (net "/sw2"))
 (segment (start 161.274314 41.6) (end 161.8 41.6) (width 0.2) (layer "F.Cu") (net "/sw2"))
 (segment (start 159.464314 43.41) (end 161.274314 41.6) (width 0.2) (layer "F.Cu") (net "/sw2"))
 (segment (start 172.2 42.93) (end 172.83 42.3) (width 0.2) (layer "F.Cu") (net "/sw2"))
 (segment (start 153.55 43.41) (end 159.464314 43.41) (width 0.2) (layer "F.Cu") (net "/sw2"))
 (segment (start 172.2 44.1) (end 172.2 42.93) (width 0.2) (layer "F.Cu") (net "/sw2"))
 (via (at 161.8 41.6) (size 0.6) (drill 0.3) (layers "F.Cu" "B.Cu") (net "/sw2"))
 (segment (start 161.8 41.6) (end 161.8 42.1) (width 0.2) (layer "B.Cu") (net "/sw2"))
 (segment (start 161.8 42.1) (end 162 42.3) (width 0.2) (layer "B.Cu") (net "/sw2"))
 (segment (start 162 42.3) (end 162 44.1) (width 0.2) (layer "B.Cu") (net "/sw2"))
 (segment (start 162.03 56.1) (end 165.3 56.1) (width 0.2) (layer "F.Cu") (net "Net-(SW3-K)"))
 (segment (start 165.3 56) (end 165.805 55.495) (width 0.2) (layer "F.Cu") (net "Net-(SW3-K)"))
 (segment (start 165.3 56.1) (end 165.3 56) (width 0.2) (layer "F.Cu") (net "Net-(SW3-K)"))
 (segment (start 160.73 54.8) (end 162.03 56.1) (width 0.2) (layer "F.Cu") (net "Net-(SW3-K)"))
 (segment (start 165.805 55.495) (end 165.805 54.1) (width 0.2) (layer "F.Cu") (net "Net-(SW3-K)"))
 (segment (start 175.37 45.23) (end 175.37 42.3) (width 0.2) (layer "F.Cu") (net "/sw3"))
 (segment (start 173.1 47.5) (end 175.37 45.23) (width 0.2) (layer "F.Cu") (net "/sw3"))
 (segment (start 186.6 51.6) (end 183 51.6) (width 0.2) (layer "F.Cu") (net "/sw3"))
 (segment (start 183 51.6) (end 183.05 51.55) (width 0.2) (layer "F.Cu") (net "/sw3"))
 (segment (start 166.409745 47.625) (end 167.590255 47.625) (width 0.2) (layer "F.Cu") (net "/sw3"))
 (segment (start 168.315255 46.9) (end 170.5 46.9) (width 0.2) (layer "F.Cu") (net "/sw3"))
 (segment (start 156.54 46.9) (end 165.684745 46.9) (width 0.2) (layer "F.Cu") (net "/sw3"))
 (segment (start 183.05 46.15) (end 181 44.1) (width 0.2) (layer "F.Cu") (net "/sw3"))
 (segment (start 165.684745 46.9) (end 166.409745 47.625) (width 0.2) (layer "F.Cu") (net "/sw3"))
 (segment (start 167.590255 47.625) (end 168.315255 46.9) (width 0.2) (layer "F.Cu") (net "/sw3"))
 (segment (start 188.6 49.6) (end 186.6 51.6) (width 0.2) (layer "F.Cu") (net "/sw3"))
 (segment (start 183.05 51.55) (end 183.05 46.15) (width 0.2) (layer "F.Cu") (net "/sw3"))
 (segment (start 156.1 47.34) (end 156.54 46.9) (width 0.2) (layer "F.Cu") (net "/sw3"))
 (segment (start 170.5 46.9) (end 171.2 47.6) (width 0.2) (layer "F.Cu") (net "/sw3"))
 (via (at 173.1 47.5) (size 0.6) (drill 0.3) (layers "F.Cu" "B.Cu") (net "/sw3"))
 (via (at 171.2 47.6) (size 0.6) (drill 0.3) (layers "F.Cu" "B.Cu") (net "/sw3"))
 (via (at 188.6 49.6) (size 0.6) (drill 0.3) (layers "F.Cu" "B.Cu") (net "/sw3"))
 (segment (start 177.17 44.1) (end 175.37 42.3) (width 0.2) (layer "B.Cu") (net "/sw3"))
 (segment (start 188.745 49.6) (end 188.6 49.6) (width 0.2) (layer "B.Cu") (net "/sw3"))
 (segment (start 191.4 52.255) (end 188.745 49.6) (width 0.2) (layer "B.Cu") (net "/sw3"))
 (segment (start 173 47.6) (end 173.1 47.5) (width 0.2) (layer "B.Cu") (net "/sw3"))
 (segment (start 181 44.1) (end 177.17 44.1) (width 0.2) (layer "B.Cu") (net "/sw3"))
 (segment (start 171.2 47.6) (end 173 47.6) (width 0.2) (layer "B.Cu") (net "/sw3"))
 (segment (start 184.1 55.505) (end 185.305 54.3) (width 0.2) (layer "F.Cu") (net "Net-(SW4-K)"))
 (segment (start 179.73 54.8) (end 181.33 56.4) (width 0.2) (layer "F.Cu") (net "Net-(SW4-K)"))
 (segment (start 181.33 56.4) (end 184.1 56.4) (width 0.2) (layer "F.Cu") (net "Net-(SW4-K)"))
 (segment (start 184.1 56.4) (end 184.1 55.505) (width 0.2) (layer "F.Cu") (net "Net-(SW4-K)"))
 (segment (start 179.71 55.1) (end 179.73 55.08) (width 0.2) (layer "F.Cu") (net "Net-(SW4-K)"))
 (segment (start 150.4 47.3) (end 152.2 47.3) (width 0.2) (layer "F.Cu") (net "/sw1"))
 (segment (start 170.29 42.3) (end 161.14 42.3) (width 0.2) (layer "F.Cu") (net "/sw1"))
 (segment (start 161.14 42.3) (end 157.25 46.19) (width 0.2) (layer "F.Cu") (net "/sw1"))
 (segment (start 138.055 42) (end 140.155 44.1) (width 0.2) (layer "F.Cu") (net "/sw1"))
 (segment (start 147.2 48.3) (end 149.4 48.3) (width 0.2) (layer "F.Cu") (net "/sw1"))
 (segment (start 149.4 48.3) (end 150.4 47.3) (width 0.2) (layer "F.Cu") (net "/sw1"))
 (segment (start 157.25 46.19) (end 153.31 46.19) (width 0.2) (layer "F.Cu") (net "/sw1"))
 (segment (start 143 44.1) (end 147.2 48.3) (width 0.2) (layer "F.Cu") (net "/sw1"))
 (segment (start 153.31 46.19) (end 152.2 47.3) (width 0.2) (layer "F.Cu") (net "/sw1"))
 (segment (start 140.155 44.1) (end 143 44.1) (width 0.2) (layer "F.Cu") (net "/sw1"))
 (segment (start 143.05 56.4) (end 145.36 56.4) (width 0.2) (layer "F.Cu") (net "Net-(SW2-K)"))
 (segment (start 145.36 56.4) (end 146.56 55.2) (width 0.2) (layer "F.Cu") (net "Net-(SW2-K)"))
 (segment (start 141.73 55.08) (end 143.05 56.4) (width 0.2) (layer "F.Cu") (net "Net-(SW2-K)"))
 (segment (start 194.17 42.3) (end 193.1 43.37) (width 0.2) (layer "F.Cu") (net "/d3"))
 (segment (start 187.845 53.055) (end 187.845 54.3) (width 0.2) (layer "F.Cu") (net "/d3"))
 (segment (start 193.1 47.8) (end 187.845 53.055) (width 0.2) (layer "F.Cu") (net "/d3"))
 (segment (start 193.1 43.37) (end 193.1 47.8) (width 0.2) (layer "F.Cu") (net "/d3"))
 (segment (start 207.244999 54.000001) (end 207.244999 46.344999) (width 0.2) (layer "F.Cu") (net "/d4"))
 (segment (start 202.5 44.4) (end 200.4 42.3) (width 0.2) (layer "F.Cu") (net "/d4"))
 (segment (start 206.445 54.8) (end 207.244999 54.000001) (width 0.2) (layer "F.Cu") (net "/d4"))
 (segment (start 200.4 42.3) (end 196.71 42.3) (width 0.2) (layer "F.Cu") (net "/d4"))
 (segment (start 207.244999 46.344999) (end 205.3 44.4) (width 0.2) (layer "F.Cu") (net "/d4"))
 (segment (start 205.3 44.4) (end 202.5 44.4) (width 0.2) (layer "F.Cu") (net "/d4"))
 (segment (start 169.6 56.1) (end 169.6 55.355) (width 0.2) (layer "F.Cu") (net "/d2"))
 (segment (start 185.182207 52.867158) (end 184.799365 53.25) (width 0.2) (layer "F.Cu") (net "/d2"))
 (segment (start 187.467157 52.867158) (end 185.182207 52.867158) (width 0.2) (layer "F.Cu") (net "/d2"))
 (segment (start 191.63 42.3) (end 192.7 43.37) (width 0.2) (layer "F.Cu") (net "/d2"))
 (segment (start 169.6 55.355) (end 168.345 54.1) (width 0.2) (layer "F.Cu") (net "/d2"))
 (segment (start 173.3 55.350635) (end 172.550635 56.1) (width 0.2) (layer "F.Cu") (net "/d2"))
 (segment (start 184.799365 53.25) (end 175.386497 53.25) (width 0.2) (layer "F.Cu") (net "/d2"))
 (segment (start 192.7 47.634314) (end 187.467157 52.867158) (width 0.2) (layer "F.Cu") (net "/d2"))
 (segment (start 192.7 43.37) (end 192.7 47.634314) (width 0.2) (layer "F.Cu") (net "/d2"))
 (segment (start 172.550635 56.1) (end 169.6 56.1) (width 0.2) (layer "F.Cu") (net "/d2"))
 (segment (start 175.386497 53.25) (end 173.3 55.336497) (width 0.2) (layer "F.Cu") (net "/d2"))
 (segment (start 173.3 55.336497) (end 173.3 55.350635) (width 0.2) (layer "F.Cu") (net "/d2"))
 (segment (start 189.09 42.3) (end 189.2 42.3) (width 0.2) (layer "F.Cu") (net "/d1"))
 (segment (start 174.65 52.85) (end 174.045 53.455) (width 0.2) (layer "F.Cu") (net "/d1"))
 (segment (start 171.744365 53.455) (end 171.289365 53) (width 0.2) (layer "F.Cu") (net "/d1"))
 (segment (start 171.289365 53) (end 150.845 53) (width 0.2) (layer "F.Cu") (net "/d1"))
 (segment (start 150.845 53) (end 149.445 54.4) (width 0.2) (layer "F.Cu") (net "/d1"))
 (segment (start 184.932842 52.467158) (end 184.55 52.85) (width 0.2) (layer "F.Cu") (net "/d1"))
 (segment (start 189.2 42.3) (end 192.3 45.4) (width 0.2) (layer "F.Cu") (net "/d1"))
 (segment (start 174.045 53.455) (end 171.744365 53.455) (width 0.2) (layer "F.Cu") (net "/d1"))
 (segment (start 187.301471 52.467158) (end 184.932842 52.467158) (width 0.2) (layer "F.Cu") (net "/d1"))
 (segment (start 192.3 45.4) (end 192.3 47.468628) (width 0.2) (layer "F.Cu") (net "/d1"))
 (segment (start 192.3 47.468628) (end 187.301471 52.467158) (width 0.2) (layer "F.Cu") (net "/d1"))
 (segment (start 184.55 52.85) (end 174.65 52.85) (width 0.2) (layer "F.Cu") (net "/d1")))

